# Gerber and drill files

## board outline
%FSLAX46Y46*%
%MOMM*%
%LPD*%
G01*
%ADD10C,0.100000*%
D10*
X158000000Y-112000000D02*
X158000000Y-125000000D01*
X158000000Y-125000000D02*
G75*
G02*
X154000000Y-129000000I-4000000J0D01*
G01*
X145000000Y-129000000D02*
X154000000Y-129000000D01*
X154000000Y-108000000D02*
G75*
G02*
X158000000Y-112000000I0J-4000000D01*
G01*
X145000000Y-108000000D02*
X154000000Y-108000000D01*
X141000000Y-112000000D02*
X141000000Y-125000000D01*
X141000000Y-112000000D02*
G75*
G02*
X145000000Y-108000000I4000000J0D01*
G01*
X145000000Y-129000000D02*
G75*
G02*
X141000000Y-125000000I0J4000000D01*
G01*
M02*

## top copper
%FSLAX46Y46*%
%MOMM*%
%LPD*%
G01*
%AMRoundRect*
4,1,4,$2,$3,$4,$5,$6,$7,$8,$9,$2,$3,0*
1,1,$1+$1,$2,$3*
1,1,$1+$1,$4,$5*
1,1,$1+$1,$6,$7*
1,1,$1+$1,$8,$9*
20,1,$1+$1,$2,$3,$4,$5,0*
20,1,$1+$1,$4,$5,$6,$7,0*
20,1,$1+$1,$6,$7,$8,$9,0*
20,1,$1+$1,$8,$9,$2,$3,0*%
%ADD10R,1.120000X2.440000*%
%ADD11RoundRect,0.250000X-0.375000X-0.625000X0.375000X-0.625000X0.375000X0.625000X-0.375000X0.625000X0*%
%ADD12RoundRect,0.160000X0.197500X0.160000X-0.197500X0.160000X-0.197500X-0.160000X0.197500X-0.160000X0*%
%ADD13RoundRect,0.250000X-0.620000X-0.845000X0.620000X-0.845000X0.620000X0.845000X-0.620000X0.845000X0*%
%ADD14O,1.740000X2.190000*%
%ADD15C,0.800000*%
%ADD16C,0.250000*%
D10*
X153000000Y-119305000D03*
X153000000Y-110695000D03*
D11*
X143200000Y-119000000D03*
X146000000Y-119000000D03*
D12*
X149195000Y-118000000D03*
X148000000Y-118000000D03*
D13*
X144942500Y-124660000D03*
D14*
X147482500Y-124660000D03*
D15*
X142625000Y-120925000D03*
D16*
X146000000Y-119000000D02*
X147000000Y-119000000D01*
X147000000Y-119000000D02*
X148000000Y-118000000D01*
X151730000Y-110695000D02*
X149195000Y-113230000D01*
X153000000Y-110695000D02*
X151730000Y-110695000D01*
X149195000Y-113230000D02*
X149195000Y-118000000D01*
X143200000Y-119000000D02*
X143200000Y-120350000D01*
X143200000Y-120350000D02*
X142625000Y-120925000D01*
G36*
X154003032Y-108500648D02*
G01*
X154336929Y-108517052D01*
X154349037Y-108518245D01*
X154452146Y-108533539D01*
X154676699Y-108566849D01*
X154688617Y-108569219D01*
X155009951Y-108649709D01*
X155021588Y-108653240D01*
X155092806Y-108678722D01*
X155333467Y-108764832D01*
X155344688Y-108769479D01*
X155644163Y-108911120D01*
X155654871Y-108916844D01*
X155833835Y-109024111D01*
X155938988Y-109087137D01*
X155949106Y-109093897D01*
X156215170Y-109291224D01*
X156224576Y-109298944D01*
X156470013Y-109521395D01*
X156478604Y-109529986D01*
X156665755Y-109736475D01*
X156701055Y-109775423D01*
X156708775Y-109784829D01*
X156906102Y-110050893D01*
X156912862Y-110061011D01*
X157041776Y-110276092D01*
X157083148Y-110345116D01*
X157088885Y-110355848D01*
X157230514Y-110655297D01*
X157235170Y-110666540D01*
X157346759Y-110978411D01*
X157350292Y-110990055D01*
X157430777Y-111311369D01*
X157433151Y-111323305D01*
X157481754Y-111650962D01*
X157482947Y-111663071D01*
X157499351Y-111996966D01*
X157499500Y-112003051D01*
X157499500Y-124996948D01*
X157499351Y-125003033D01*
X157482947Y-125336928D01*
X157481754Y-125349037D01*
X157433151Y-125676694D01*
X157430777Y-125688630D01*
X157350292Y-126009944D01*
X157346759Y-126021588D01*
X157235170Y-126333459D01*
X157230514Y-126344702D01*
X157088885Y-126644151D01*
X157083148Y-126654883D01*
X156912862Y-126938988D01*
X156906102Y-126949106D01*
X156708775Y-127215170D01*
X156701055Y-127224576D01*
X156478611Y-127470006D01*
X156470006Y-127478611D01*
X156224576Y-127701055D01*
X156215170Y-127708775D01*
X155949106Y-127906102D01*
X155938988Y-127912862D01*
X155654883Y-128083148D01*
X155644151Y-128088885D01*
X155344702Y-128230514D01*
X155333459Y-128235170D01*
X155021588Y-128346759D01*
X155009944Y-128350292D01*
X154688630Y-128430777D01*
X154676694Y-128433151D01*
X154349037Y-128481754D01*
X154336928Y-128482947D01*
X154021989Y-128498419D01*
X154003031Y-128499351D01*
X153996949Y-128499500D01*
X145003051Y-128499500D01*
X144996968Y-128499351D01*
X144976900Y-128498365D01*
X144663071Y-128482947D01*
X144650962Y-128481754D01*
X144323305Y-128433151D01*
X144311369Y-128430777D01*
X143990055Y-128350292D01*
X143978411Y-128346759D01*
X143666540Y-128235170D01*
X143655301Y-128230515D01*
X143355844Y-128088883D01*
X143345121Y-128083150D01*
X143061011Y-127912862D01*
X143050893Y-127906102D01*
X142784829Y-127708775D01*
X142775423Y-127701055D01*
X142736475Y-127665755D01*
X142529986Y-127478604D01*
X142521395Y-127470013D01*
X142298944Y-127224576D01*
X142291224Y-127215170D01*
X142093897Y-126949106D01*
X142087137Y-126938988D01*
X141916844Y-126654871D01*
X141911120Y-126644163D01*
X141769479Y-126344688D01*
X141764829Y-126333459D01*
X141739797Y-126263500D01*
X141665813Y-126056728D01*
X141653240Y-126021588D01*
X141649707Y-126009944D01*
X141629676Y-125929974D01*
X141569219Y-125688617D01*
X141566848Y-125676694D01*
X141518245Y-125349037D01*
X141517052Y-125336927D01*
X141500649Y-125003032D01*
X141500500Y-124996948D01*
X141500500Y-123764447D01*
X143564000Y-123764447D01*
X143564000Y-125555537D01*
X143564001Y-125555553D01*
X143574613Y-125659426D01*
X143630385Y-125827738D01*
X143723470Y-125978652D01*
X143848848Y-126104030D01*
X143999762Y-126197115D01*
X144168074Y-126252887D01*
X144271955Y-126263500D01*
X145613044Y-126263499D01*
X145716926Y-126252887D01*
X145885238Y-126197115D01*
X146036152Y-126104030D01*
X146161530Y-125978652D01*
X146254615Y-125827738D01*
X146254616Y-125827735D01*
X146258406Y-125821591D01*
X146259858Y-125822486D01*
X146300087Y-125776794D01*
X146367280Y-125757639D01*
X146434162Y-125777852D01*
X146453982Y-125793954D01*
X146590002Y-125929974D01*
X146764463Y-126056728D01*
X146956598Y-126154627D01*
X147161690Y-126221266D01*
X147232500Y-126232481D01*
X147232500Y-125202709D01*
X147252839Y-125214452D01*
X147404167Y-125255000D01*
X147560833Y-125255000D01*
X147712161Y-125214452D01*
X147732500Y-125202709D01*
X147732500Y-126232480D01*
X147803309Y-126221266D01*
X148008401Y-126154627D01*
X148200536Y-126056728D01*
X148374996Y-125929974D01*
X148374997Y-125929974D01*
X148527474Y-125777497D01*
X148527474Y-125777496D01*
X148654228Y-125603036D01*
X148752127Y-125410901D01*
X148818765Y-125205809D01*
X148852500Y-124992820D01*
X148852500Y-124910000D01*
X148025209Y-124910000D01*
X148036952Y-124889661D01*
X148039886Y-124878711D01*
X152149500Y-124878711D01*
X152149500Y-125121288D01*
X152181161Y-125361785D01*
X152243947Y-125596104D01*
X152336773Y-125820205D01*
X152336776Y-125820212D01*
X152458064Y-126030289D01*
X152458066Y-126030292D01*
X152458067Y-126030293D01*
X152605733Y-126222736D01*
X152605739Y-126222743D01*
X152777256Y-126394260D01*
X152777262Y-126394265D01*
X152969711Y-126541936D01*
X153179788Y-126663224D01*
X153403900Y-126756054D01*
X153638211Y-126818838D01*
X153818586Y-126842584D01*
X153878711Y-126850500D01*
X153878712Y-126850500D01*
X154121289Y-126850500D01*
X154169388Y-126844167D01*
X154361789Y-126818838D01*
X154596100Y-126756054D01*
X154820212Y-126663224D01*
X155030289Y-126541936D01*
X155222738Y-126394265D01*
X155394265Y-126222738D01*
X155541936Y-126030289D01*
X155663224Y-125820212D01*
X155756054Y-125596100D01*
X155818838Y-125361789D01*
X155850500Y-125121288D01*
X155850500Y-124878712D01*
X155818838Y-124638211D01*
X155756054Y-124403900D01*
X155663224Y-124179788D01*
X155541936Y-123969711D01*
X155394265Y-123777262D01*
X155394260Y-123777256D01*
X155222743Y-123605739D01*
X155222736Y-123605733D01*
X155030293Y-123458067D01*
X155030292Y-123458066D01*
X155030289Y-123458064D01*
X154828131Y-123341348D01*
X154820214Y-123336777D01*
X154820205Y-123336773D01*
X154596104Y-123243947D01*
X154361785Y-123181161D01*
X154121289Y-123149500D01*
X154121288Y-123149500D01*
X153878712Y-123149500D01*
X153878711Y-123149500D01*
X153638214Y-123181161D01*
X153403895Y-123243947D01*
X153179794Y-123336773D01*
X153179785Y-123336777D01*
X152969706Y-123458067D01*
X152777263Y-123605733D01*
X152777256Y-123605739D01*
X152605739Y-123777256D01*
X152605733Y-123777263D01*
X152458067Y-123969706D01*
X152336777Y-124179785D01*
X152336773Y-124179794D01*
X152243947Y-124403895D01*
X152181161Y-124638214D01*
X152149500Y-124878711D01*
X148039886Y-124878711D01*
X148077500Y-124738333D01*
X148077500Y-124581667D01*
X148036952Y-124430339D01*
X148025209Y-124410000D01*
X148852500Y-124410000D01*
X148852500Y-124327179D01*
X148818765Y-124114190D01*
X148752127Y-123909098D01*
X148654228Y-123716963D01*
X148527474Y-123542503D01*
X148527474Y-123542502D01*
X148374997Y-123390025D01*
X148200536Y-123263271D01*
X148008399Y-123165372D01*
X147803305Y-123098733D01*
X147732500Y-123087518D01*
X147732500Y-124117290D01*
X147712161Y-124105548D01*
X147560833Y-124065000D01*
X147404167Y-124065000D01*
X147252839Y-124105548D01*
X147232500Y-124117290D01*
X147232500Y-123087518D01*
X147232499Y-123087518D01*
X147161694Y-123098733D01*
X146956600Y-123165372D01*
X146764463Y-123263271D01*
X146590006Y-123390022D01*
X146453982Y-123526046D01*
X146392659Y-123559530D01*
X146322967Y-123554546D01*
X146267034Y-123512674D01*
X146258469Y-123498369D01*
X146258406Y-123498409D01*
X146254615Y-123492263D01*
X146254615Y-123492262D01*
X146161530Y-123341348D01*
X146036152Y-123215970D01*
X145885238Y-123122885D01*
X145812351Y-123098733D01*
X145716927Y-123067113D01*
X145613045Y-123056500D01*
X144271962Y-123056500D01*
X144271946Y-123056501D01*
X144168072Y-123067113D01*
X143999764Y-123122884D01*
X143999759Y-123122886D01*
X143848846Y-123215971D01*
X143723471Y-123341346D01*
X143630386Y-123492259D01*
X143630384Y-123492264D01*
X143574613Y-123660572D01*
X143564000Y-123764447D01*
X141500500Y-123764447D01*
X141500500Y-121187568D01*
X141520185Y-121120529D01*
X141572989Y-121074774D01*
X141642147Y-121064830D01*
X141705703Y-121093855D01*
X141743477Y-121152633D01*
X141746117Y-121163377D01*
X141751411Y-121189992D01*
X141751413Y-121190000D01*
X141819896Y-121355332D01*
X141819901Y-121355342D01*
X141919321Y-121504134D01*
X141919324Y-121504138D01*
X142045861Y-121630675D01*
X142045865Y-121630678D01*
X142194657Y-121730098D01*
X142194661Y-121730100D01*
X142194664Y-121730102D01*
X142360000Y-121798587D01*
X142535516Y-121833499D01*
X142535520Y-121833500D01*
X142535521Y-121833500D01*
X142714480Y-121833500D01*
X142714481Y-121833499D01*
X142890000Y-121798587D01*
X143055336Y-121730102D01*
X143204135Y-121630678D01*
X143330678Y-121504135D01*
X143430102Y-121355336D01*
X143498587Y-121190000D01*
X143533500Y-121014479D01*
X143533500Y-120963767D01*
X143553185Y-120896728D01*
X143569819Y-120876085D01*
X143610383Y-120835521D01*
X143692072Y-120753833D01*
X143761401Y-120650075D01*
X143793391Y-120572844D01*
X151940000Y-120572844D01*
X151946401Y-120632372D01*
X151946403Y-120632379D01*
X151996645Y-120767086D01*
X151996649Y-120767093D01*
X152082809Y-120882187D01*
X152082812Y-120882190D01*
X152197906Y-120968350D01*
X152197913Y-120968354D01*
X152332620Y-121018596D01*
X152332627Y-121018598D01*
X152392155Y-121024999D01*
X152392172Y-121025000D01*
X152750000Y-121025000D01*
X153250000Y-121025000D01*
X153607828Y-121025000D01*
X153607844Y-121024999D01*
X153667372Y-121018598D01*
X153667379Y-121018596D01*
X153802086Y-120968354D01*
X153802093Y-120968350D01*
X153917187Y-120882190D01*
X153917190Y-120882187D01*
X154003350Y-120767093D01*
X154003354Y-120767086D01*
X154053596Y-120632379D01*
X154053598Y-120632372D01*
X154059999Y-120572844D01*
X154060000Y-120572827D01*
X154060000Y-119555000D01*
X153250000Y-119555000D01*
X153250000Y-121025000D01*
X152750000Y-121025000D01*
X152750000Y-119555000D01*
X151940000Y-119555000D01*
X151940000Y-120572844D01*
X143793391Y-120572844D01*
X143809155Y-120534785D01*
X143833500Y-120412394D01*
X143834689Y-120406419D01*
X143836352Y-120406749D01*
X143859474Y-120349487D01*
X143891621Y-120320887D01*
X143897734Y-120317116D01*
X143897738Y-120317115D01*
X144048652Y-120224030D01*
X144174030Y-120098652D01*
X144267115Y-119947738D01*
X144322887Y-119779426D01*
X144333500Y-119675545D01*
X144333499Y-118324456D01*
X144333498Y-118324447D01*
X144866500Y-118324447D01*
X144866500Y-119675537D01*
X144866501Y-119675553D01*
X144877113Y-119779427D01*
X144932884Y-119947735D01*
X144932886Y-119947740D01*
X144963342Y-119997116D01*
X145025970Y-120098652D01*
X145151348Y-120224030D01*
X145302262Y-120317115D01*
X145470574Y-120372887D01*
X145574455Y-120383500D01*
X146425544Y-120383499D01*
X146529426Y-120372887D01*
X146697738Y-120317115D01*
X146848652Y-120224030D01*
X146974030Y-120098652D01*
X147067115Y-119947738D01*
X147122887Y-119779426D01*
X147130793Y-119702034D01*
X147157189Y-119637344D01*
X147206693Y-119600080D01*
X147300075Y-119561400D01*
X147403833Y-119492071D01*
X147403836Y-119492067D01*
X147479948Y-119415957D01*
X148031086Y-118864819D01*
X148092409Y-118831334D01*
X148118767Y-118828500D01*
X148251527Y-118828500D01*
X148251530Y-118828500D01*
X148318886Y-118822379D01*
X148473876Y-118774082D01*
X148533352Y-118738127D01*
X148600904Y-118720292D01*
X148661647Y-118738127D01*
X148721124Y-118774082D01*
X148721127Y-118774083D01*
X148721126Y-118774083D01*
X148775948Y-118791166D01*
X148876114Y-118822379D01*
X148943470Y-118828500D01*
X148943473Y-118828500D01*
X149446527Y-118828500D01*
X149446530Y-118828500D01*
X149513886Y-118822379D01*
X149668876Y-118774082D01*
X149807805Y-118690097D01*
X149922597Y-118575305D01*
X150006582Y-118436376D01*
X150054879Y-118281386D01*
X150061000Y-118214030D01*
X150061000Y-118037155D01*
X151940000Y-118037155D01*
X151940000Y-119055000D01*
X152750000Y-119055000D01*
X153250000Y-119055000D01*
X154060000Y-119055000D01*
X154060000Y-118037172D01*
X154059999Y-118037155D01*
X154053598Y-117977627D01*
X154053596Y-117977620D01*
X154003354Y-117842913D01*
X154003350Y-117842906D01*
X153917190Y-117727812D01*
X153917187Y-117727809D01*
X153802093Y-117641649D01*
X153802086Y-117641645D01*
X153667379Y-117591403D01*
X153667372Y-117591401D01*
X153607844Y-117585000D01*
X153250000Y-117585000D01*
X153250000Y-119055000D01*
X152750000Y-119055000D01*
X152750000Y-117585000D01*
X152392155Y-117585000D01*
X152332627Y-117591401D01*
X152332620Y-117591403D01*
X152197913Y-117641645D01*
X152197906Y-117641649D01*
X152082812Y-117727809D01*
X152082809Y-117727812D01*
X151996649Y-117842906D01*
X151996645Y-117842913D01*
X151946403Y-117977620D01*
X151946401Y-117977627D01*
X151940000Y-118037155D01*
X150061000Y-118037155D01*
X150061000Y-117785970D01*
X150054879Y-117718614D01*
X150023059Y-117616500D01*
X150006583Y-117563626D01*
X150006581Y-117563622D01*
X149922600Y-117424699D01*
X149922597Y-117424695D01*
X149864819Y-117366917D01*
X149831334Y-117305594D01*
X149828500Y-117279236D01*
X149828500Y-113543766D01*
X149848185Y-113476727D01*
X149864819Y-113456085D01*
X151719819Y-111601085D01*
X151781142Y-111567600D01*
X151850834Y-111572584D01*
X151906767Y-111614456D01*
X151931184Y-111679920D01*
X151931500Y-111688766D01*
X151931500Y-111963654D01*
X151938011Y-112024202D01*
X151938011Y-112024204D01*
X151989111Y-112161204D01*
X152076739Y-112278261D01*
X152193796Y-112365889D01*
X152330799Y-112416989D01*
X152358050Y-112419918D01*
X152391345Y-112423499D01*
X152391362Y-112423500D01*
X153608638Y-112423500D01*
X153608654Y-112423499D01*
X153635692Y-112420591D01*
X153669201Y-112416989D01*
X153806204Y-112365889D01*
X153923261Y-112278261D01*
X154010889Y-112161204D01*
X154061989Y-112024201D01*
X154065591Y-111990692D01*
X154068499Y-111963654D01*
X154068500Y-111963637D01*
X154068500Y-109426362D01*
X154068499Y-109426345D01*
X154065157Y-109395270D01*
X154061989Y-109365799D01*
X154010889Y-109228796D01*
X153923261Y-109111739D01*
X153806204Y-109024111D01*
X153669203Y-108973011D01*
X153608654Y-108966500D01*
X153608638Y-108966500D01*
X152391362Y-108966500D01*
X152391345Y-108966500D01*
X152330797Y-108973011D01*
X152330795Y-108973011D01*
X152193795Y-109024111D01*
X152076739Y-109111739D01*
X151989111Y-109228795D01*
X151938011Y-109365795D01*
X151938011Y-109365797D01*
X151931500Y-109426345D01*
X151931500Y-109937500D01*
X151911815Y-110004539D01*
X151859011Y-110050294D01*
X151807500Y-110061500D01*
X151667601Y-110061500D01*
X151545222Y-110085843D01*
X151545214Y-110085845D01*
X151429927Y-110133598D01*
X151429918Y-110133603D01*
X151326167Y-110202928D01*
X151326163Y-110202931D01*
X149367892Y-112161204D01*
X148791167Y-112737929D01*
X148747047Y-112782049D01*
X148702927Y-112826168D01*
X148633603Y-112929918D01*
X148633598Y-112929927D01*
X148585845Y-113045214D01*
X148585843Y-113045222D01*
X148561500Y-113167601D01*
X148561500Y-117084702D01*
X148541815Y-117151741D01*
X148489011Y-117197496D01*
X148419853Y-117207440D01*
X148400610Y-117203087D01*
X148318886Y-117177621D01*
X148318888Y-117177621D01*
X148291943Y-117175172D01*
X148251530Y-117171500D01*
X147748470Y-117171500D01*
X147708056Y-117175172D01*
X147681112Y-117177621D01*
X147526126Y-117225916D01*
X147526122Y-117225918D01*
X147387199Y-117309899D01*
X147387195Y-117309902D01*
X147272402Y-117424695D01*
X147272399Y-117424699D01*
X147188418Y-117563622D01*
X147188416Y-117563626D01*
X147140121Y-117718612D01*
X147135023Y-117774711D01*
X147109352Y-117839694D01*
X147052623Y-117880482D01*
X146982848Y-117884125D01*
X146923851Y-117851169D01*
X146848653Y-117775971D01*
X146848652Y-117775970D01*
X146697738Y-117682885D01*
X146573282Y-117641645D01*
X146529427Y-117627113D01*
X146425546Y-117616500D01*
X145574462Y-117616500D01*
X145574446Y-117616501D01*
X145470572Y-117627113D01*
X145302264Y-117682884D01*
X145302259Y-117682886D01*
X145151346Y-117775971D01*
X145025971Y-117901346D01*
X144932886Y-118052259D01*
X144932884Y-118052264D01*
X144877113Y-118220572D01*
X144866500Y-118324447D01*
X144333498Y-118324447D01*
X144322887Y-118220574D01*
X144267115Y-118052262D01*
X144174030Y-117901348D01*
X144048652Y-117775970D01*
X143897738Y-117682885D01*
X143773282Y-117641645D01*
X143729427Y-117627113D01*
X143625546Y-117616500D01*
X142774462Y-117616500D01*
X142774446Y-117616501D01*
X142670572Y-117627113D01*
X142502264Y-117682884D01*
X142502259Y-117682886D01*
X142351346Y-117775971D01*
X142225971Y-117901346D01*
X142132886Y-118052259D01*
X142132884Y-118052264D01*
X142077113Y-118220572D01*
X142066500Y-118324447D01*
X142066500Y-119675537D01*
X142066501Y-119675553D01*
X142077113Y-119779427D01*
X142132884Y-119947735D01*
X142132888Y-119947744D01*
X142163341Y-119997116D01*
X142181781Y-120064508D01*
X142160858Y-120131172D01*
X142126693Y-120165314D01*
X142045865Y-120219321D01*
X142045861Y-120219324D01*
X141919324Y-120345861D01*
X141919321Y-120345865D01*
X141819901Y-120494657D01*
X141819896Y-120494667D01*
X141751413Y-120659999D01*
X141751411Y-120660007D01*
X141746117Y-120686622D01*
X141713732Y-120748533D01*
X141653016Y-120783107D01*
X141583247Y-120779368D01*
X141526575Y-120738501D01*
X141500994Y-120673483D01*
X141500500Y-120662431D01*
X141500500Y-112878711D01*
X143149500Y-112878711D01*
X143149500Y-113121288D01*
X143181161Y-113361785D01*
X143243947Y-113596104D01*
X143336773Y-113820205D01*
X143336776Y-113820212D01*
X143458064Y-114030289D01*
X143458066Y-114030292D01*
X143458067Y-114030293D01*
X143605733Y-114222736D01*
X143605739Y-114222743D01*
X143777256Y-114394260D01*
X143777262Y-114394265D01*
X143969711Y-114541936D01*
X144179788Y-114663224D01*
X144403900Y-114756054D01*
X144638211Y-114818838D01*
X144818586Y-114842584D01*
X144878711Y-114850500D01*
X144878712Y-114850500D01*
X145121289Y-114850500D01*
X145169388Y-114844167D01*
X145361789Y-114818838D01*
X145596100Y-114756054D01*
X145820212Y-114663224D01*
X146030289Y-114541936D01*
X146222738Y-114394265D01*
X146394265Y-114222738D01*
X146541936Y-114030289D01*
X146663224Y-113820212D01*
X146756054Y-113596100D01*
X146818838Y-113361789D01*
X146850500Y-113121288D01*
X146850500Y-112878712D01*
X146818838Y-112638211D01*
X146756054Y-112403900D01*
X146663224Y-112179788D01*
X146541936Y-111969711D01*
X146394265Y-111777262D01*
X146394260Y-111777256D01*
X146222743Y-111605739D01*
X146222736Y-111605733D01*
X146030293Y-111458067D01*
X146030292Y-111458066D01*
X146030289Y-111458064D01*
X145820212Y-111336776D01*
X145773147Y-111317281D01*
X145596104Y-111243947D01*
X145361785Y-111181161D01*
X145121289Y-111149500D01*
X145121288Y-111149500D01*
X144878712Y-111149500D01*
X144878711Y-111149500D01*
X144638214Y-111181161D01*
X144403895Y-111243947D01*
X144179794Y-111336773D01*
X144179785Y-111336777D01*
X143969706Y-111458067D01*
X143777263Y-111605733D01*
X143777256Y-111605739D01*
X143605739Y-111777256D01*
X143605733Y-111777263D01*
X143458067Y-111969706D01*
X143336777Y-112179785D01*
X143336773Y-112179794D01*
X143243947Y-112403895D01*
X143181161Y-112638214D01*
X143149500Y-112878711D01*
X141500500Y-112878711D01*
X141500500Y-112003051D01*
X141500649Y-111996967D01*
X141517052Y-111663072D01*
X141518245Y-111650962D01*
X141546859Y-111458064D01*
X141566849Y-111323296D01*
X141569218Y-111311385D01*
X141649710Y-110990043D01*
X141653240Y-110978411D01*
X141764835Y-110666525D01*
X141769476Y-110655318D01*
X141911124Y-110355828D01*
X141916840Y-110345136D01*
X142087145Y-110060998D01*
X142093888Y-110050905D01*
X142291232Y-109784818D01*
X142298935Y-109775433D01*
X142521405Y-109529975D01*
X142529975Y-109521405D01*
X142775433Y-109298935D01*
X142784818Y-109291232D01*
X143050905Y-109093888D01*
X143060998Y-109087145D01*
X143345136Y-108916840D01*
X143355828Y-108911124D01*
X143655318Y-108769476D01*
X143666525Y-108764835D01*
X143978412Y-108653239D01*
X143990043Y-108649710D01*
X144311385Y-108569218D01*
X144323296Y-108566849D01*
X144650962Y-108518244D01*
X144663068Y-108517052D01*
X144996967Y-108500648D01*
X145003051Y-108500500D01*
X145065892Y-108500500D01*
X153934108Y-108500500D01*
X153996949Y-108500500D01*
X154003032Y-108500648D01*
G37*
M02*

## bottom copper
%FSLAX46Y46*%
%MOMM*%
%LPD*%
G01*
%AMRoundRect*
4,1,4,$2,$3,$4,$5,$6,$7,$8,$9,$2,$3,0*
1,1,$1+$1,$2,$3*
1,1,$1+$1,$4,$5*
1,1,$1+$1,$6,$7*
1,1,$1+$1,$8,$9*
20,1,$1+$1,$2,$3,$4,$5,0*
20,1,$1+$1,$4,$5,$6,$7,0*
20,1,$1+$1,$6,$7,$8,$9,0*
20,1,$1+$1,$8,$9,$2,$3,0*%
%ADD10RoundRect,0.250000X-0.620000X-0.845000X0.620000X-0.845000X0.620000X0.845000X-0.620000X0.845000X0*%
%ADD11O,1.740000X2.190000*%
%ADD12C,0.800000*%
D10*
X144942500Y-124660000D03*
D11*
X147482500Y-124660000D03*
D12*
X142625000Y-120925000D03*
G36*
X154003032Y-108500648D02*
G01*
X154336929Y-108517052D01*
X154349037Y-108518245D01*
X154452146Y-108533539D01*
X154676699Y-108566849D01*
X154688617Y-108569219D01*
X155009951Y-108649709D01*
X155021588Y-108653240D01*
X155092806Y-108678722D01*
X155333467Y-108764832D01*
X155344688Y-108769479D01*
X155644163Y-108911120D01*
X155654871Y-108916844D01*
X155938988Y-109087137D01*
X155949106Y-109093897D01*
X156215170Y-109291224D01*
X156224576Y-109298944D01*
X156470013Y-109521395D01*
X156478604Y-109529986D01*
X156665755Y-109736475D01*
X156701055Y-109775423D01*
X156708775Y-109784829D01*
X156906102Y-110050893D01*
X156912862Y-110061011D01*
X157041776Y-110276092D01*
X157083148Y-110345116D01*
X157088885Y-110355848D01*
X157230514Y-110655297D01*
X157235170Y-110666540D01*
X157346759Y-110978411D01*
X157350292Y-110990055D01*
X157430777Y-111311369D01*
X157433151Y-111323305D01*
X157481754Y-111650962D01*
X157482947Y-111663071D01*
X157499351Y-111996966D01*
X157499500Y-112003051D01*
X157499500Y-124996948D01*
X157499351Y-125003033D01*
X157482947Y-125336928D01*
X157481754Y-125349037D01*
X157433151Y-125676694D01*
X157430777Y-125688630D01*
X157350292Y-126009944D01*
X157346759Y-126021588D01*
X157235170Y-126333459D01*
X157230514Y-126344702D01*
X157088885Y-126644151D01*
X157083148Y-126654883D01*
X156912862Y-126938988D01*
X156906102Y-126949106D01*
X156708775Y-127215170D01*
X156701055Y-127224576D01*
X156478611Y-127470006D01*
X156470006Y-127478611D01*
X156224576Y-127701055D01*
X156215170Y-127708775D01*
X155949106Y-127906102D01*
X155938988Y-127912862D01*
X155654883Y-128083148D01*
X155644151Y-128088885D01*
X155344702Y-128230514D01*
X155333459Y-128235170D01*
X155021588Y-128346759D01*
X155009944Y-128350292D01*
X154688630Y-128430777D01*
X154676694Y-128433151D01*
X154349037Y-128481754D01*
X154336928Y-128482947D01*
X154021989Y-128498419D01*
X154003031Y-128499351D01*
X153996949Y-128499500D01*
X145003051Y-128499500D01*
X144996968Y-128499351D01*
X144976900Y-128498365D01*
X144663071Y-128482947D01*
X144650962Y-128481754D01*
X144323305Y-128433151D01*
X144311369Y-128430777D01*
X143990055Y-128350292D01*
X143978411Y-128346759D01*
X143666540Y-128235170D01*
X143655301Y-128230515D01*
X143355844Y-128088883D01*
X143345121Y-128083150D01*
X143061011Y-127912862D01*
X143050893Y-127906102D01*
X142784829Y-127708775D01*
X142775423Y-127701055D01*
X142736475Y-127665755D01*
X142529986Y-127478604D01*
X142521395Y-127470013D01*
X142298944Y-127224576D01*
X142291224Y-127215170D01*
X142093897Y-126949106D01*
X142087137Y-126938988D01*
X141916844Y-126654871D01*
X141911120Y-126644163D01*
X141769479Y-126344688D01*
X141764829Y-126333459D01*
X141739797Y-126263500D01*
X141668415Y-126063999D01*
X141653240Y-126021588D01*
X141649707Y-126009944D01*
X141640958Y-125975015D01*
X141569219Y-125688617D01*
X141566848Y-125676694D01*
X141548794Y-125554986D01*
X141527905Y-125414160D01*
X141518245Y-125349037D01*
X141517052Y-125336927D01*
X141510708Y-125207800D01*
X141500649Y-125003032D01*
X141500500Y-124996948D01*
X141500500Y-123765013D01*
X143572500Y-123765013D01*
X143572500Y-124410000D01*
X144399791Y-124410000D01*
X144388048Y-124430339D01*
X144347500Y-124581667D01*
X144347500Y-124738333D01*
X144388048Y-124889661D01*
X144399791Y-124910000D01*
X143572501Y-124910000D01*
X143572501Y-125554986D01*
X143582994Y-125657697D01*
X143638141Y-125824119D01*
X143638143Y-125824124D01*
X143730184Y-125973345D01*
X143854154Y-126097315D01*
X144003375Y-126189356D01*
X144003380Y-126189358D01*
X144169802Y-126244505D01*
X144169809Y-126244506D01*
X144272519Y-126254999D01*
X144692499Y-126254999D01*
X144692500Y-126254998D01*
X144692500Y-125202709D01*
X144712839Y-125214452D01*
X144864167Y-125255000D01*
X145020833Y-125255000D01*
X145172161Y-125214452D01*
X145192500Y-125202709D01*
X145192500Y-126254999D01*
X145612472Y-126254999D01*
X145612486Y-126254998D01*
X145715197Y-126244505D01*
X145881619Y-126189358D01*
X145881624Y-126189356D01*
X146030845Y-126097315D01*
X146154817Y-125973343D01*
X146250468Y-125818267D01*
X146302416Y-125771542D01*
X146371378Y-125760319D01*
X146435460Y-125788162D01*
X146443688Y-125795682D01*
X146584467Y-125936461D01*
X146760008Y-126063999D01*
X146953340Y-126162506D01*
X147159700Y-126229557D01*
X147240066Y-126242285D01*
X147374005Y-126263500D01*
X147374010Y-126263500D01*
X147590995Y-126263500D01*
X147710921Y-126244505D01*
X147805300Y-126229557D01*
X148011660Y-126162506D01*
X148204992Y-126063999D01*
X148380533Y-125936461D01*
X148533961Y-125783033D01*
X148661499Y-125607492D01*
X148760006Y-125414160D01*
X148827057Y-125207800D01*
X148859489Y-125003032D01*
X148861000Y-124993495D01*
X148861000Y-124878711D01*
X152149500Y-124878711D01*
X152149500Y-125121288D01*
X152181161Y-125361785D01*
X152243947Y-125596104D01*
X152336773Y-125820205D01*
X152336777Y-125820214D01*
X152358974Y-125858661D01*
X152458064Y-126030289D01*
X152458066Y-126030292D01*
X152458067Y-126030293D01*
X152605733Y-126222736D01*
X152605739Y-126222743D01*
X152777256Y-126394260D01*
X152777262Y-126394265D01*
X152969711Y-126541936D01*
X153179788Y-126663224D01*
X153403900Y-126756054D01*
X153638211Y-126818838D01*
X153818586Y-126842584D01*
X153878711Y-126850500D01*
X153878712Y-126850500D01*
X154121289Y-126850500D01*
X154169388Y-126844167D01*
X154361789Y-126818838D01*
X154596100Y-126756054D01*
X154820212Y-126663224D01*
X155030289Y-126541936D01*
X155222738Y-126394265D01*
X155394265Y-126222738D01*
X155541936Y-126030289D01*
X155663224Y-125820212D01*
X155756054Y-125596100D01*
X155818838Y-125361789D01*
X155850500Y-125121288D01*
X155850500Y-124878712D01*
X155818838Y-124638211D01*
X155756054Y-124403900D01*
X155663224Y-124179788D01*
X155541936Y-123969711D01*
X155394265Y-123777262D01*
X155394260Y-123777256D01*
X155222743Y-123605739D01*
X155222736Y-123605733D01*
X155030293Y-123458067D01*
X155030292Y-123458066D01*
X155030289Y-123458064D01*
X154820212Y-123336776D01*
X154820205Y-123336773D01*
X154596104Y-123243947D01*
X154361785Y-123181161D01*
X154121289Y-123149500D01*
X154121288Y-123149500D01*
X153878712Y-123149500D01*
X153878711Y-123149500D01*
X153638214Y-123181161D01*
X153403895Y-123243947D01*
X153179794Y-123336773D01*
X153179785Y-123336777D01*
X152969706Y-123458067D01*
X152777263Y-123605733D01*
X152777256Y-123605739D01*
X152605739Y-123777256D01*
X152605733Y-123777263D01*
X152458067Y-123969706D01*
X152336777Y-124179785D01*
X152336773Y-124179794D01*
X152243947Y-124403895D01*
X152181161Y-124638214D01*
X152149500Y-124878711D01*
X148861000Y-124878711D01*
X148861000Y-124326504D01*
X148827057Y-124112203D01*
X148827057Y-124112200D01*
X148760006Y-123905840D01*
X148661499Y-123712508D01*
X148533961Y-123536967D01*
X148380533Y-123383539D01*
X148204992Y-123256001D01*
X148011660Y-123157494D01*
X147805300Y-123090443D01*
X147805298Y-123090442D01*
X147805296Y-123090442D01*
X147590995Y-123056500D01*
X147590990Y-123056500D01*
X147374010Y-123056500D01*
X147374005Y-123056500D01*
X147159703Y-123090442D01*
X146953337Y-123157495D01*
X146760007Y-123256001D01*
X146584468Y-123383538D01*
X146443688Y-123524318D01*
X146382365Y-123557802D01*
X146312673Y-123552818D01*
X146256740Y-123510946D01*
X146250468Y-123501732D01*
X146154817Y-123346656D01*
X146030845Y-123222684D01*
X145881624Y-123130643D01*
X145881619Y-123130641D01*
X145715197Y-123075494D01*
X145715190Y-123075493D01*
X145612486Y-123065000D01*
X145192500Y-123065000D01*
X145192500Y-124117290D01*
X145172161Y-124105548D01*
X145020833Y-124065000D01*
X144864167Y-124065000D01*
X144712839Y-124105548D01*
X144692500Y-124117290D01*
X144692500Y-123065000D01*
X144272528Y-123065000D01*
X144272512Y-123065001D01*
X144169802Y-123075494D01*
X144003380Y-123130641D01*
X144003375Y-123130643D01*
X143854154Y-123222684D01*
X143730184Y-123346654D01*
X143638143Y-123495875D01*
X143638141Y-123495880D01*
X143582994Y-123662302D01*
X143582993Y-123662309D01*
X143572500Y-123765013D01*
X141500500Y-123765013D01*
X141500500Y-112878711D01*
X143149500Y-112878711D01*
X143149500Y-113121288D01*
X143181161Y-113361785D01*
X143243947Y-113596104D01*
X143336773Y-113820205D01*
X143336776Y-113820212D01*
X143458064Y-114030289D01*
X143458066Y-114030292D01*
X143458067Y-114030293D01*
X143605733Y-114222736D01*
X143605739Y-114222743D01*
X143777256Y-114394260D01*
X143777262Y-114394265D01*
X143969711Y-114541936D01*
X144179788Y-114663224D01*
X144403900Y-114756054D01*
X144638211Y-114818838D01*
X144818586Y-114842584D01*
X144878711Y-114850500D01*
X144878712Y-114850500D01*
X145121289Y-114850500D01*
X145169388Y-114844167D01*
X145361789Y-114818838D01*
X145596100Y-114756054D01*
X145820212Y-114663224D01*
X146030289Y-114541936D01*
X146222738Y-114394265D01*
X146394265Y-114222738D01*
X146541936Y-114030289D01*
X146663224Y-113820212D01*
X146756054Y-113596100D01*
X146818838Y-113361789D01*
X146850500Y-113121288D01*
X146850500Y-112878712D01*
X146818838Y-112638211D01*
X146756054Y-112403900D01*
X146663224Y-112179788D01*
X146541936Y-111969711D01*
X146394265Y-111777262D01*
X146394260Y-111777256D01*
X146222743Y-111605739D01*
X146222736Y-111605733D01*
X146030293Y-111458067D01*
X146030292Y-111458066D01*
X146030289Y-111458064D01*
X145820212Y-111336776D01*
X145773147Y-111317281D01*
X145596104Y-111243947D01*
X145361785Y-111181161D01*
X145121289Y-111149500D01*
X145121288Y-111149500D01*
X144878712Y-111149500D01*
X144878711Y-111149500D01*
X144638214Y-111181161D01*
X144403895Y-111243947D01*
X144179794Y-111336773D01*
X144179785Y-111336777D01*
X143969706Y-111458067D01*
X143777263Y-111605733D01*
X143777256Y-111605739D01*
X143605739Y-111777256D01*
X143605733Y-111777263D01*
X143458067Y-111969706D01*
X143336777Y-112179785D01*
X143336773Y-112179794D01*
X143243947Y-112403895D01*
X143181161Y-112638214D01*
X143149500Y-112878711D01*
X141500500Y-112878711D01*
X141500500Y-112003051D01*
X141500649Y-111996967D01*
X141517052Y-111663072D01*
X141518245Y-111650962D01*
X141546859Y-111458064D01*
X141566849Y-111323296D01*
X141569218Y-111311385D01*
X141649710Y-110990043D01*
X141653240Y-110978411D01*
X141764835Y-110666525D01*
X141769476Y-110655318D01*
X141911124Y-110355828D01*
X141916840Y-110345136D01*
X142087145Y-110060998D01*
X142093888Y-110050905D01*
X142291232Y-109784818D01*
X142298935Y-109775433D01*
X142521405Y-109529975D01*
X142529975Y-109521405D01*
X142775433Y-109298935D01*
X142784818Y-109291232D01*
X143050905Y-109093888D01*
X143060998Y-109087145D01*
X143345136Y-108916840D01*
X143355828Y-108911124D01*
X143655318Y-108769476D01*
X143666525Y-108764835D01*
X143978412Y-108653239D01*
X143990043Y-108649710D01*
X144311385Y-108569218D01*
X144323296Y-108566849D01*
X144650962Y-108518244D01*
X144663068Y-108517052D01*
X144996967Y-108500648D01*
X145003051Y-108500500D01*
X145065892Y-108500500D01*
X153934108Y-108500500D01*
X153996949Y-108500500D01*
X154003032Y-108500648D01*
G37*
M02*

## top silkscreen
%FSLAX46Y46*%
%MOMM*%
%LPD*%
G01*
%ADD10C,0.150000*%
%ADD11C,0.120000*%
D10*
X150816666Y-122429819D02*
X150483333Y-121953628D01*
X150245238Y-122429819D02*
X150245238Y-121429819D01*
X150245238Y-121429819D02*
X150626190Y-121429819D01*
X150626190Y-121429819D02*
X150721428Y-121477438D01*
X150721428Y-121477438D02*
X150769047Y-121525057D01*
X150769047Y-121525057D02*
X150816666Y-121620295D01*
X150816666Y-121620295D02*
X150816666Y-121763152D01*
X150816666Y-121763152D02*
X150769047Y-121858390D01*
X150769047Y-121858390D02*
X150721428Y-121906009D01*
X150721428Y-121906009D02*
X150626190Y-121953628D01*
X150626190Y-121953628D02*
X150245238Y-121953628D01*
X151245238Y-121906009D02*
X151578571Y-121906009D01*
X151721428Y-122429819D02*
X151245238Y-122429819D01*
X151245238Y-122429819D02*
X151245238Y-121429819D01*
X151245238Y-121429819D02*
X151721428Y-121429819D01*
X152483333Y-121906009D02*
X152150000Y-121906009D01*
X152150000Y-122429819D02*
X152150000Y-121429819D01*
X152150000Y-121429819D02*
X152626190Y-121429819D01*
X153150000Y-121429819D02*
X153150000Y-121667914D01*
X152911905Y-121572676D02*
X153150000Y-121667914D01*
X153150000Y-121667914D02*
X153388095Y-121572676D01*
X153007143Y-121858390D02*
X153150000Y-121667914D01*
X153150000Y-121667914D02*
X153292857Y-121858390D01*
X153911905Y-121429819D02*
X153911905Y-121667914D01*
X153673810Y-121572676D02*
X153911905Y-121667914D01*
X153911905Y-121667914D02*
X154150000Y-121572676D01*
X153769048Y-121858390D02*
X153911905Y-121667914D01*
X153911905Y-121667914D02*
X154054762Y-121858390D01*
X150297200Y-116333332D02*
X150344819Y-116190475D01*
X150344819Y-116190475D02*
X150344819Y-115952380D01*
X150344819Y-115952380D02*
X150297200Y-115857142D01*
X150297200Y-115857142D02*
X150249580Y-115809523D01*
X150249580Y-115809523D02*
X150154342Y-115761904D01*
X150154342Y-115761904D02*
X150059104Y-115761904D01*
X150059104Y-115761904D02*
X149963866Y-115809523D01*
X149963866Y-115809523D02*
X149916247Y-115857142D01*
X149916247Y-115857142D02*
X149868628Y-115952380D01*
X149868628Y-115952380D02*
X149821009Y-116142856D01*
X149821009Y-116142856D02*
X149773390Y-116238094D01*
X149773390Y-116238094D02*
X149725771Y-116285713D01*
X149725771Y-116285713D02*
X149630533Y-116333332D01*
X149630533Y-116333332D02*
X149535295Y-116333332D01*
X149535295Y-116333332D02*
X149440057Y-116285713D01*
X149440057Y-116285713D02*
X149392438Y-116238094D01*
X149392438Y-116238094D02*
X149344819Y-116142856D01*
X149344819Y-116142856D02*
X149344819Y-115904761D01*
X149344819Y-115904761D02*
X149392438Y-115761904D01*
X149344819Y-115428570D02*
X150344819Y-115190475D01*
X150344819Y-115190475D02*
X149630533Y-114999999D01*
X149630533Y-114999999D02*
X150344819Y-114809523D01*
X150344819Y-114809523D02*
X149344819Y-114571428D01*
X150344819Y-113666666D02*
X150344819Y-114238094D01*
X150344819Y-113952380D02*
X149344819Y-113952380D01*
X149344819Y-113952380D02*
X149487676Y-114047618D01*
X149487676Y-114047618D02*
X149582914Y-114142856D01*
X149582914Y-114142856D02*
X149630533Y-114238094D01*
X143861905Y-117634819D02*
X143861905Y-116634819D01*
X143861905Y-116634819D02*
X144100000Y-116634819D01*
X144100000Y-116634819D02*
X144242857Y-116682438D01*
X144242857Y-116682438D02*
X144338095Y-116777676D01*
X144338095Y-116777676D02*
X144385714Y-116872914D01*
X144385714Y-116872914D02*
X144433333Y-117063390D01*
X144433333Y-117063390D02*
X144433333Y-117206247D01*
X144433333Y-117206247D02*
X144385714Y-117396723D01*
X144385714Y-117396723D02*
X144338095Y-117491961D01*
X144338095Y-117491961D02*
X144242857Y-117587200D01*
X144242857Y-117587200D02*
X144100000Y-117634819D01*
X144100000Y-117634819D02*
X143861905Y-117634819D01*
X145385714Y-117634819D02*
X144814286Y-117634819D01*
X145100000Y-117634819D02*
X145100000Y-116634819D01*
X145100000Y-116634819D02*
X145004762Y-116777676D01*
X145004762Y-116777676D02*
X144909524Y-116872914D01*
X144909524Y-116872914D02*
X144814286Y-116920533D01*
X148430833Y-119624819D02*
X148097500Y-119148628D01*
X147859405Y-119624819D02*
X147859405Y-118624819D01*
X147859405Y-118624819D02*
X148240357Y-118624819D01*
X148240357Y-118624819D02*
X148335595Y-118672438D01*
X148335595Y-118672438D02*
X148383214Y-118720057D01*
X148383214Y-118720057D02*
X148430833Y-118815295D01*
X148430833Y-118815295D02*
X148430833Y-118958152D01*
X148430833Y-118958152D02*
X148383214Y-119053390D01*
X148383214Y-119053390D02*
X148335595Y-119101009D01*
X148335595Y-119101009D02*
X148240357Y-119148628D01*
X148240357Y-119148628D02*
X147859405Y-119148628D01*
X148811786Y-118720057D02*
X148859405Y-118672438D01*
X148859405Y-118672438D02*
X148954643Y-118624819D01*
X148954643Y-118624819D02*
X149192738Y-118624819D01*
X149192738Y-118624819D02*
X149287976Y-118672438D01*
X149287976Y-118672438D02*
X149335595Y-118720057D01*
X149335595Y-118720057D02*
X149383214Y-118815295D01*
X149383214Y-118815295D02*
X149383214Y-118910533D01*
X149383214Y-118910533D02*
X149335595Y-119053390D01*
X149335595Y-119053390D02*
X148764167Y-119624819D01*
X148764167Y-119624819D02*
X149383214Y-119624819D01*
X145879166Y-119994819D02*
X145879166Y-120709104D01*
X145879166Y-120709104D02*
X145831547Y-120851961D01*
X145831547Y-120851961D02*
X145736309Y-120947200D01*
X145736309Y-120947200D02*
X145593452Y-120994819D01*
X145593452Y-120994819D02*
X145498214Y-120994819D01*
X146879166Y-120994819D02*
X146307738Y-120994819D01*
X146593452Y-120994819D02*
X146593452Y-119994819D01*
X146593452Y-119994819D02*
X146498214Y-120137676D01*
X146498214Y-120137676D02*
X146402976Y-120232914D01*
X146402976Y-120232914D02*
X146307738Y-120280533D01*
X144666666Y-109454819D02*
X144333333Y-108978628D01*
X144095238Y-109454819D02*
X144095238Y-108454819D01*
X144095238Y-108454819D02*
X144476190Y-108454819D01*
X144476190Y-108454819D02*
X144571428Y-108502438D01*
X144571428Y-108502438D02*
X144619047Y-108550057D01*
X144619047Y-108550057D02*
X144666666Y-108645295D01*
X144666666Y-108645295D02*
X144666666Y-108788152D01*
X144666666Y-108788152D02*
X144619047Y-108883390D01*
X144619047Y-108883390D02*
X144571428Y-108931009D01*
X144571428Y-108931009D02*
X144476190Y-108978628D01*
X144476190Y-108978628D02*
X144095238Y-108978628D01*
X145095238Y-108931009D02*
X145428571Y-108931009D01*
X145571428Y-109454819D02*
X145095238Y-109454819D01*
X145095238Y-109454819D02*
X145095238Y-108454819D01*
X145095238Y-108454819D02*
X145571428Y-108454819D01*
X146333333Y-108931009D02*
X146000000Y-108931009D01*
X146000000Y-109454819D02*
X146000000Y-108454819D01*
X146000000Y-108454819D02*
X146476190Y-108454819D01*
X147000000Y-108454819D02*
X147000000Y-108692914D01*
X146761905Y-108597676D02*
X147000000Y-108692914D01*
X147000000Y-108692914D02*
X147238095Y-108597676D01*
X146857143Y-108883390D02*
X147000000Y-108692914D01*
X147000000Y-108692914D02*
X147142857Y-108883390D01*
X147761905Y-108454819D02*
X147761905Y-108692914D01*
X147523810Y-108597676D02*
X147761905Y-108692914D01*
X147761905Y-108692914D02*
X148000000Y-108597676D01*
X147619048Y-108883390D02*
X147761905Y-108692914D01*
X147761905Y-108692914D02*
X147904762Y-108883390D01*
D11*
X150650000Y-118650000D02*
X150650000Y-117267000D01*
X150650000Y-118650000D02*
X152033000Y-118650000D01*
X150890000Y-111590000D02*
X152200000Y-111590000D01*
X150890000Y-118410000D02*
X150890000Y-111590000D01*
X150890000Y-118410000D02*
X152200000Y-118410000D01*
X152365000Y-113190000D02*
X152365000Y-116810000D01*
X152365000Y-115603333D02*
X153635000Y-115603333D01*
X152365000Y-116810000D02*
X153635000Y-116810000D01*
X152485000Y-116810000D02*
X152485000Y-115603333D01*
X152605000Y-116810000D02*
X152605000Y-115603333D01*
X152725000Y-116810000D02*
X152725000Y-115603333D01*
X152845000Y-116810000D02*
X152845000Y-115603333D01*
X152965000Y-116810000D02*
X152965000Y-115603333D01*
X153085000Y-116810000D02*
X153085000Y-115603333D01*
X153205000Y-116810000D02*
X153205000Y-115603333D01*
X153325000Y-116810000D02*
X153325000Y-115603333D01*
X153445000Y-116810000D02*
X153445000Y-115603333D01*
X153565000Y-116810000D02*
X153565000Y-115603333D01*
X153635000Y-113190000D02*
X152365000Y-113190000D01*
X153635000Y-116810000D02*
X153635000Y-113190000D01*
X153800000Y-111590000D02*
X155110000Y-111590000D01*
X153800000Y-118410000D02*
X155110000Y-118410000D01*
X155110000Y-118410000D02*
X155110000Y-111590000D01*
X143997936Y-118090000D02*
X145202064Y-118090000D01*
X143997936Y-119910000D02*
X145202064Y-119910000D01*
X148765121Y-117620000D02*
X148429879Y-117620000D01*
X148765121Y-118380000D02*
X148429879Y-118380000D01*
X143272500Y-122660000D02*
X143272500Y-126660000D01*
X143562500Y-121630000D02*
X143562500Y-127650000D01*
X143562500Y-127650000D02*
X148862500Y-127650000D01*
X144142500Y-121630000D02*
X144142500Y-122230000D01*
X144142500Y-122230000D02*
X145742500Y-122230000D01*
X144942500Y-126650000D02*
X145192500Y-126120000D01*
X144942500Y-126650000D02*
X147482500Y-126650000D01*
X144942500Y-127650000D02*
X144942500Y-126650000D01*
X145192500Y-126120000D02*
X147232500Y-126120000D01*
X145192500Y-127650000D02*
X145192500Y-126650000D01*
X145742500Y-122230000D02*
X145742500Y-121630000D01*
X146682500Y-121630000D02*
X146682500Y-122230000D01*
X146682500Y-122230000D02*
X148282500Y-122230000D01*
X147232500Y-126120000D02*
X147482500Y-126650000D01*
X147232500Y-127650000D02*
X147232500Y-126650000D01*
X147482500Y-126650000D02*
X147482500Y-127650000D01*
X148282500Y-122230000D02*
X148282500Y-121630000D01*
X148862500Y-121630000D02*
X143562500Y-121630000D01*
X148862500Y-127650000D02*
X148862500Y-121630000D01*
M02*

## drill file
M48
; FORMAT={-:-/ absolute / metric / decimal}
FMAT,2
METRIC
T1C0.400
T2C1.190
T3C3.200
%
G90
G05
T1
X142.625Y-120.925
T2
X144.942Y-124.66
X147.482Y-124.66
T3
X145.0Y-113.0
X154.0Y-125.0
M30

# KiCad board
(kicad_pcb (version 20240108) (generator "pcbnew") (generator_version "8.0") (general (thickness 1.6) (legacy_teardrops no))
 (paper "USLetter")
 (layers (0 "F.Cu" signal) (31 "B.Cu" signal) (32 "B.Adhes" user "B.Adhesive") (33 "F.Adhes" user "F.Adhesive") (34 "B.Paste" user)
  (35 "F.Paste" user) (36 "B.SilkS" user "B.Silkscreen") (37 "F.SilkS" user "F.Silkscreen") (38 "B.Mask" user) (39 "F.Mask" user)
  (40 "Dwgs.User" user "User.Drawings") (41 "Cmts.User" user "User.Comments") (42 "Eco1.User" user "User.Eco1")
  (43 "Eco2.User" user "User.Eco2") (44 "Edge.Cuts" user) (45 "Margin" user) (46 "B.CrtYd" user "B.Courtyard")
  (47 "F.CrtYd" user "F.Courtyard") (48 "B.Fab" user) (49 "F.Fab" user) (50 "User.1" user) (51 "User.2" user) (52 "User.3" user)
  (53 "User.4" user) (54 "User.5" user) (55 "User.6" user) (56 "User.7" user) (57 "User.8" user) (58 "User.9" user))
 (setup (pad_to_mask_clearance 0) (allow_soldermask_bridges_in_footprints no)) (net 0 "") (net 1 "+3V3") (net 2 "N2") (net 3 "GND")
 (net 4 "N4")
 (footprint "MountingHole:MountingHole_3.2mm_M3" (layer "F.Cu") (at 154 125)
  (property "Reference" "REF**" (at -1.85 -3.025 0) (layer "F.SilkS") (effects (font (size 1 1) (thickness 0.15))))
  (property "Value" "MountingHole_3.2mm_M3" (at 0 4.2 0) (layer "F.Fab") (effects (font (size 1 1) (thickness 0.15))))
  (pad "" np_thru_hole circle (at 0 0) (size 3.2 3.2) (drill 3.2) (layers "*.Cu" "*.Mask")))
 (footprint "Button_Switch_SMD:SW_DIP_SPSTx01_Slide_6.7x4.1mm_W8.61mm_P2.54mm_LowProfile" (layer "F.Cu") (at 153 115 90)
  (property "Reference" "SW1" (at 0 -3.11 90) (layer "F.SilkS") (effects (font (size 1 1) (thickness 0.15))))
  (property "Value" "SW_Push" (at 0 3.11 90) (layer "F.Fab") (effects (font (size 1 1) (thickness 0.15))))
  (fp_line (start -3.65 -2.35) (end -2.267 -2.35) (stroke (width 0.12) (type solid)) (layer "F.SilkS"))
  (fp_line (start -3.65 -2.35) (end -3.65 -0.967) (stroke (width 0.12) (type solid)) (layer "F.SilkS"))
  (fp_line (start 3.41 -2.11) (end 3.41 -0.8) (stroke (width 0.12) (type solid)) (layer "F.SilkS"))
  (fp_line (start -3.41 -2.11) (end 3.41 -2.11) (stroke (width 0.12) (type solid)) (layer "F.SilkS"))
  (fp_line (start -3.41 -2.11) (end -3.41 -0.8) (stroke (width 0.12) (type solid)) (layer "F.SilkS"))
  (fp_line (start 1.81 -0.635) (end -1.81 -0.635) (stroke (width 0.12) (type solid)) (layer "F.SilkS"))
  (fp_line (start -0.603333 -0.635) (end -0.603333 0.635) (stroke (width 0.12) (type solid)) (layer "F.SilkS"))
  (fp_line (start -1.81 -0.635) (end -1.81 0.635) (stroke (width 0.12) (type solid)) (layer "F.SilkS"))
  (fp_line (start -1.81 -0.515) (end -0.603333 -0.515) (stroke (width 0.12) (type solid)) (layer "F.SilkS"))
  (fp_line (start -1.81 -0.395) (end -0.603333 -0.395) (stroke (width 0.12) (type solid)) (layer "F.SilkS"))
  (fp_line (start -1.81 -0.275) (end -0.603333 -0.275) (stroke (width 0.12) (type solid)) (layer "F.SilkS"))
  (fp_line (start -1.81 -0.155) (end -0.603333 -0.155) (stroke (width 0.12) (type solid)) (layer "F.SilkS"))
  (fp_line (start -1.81 -0.035) (end -0.603333 -0.035) (stroke (width 0.12) (type solid)) (layer "F.SilkS"))
  (fp_line (start -1.81 0.085) (end -0.603333 0.085) (stroke (width 0.12) (type solid)) (layer "F.SilkS"))
  (fp_line (start -1.81 0.205) (end -0.603333 0.205) (stroke (width 0.12) (type solid)) (layer "F.SilkS"))
  (fp_line (start -1.81 0.325) (end -0.603333 0.325) (stroke (width 0.12) (type solid)) (layer "F.SilkS"))
  (fp_line (start -1.81 0.445) (end -0.603333 0.445) (stroke (width 0.12) (type solid)) (layer "F.SilkS"))
  (fp_line (start -1.81 0.565) (end -0.603333 0.565) (stroke (width 0.12) (type solid)) (layer "F.SilkS"))
  (fp_line (start 1.81 0.635) (end 1.81 -0.635) (stroke (width 0.12) (type solid)) (layer "F.SilkS"))
  (fp_line (start -1.81 0.635) (end 1.81 0.635) (stroke (width 0.12) (type solid)) (layer "F.SilkS"))
  (fp_line (start 3.41 0.8) (end 3.41 2.11) (stroke (width 0.12) (type solid)) (layer "F.SilkS"))
  (fp_line (start -3.41 0.8) (end -3.41 2.11) (stroke (width 0.12) (type solid)) (layer "F.SilkS"))
  (fp_line (start -3.41 2.11) (end 3.41 2.11) (stroke (width 0.12) (type solid)) (layer "F.SilkS"))
  (pad "1" smd rect (at -4.305 0 90) (size 2.44 1.12) (layers "F.Cu" "F.Paste" "F.Mask") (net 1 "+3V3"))
  (pad "2" smd rect (at 4.305 0 90) (size 2.44 1.12) (layers "F.Cu" "F.Paste" "F.Mask") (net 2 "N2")))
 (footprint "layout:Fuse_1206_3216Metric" (layer "F.Cu") (at 144.6 119)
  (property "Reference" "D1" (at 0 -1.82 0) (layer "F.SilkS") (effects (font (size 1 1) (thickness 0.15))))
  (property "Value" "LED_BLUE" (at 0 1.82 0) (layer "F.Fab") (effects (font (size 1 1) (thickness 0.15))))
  (fp_line (start -0.602064 -0.91) (end 0.602064 -0.91) (stroke (width 0.12) (type solid)) (layer "F.SilkS"))
  (fp_line (start -0.602064 0.91) (end 0.602064 0.91) (stroke (width 0.12) (type solid)) (layer "F.SilkS"))
  (pad "1" smd roundrect (at -1.4 0) (size 1.25 1.75) (layers "F.Cu" "F.Paste" "F.Mask") (roundrect_rratio 0.2) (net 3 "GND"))
  (pad "2" smd roundrect (at 1.4 0) (size 1.25 1.75) (layers "F.Cu" "F.Paste" "F.Mask") (roundrect_rratio 0.2) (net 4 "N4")))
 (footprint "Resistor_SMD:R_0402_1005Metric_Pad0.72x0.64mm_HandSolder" (layer "F.Cu") (at 148.5975 118 180)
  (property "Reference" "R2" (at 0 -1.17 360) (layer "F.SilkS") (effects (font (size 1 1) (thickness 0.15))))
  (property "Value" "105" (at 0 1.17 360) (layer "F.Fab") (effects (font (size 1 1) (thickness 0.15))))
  (fp_line (start -0.167621 0.38) (end 0.167621 0.38) (stroke (width 0.12) (type solid)) (layer "F.SilkS"))
  (fp_line (start -0.167621 -0.38) (end 0.167621 -0.38) (stroke (width 0.12) (type solid)) (layer "F.SilkS"))
  (pad "1" smd roundrect (at -0.5975 0 180) (size 0.715 0.64) (layers "F.Cu" "F.Paste" "F.Mask") (roundrect_rratio 0.25) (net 2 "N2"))
  (pad "2" smd roundrect (at 0.5975 0 180) (size 0.715 0.64) (layers "F.Cu" "F.Paste" "F.Mask") (roundrect_rratio 0.25) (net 4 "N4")))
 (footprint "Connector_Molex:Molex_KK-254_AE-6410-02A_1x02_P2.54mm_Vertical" (layer "F.Cu") (at 144.9425 124.66)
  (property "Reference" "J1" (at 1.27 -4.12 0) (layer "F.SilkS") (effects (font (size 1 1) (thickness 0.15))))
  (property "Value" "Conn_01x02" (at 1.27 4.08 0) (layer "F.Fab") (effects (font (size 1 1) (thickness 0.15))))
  (fp_line (start -1.67 -2) (end -1.67 2) (stroke (width 0.12) (type solid)) (layer "F.SilkS"))
  (fp_line (start -1.38 -3.03) (end -1.38 2.99) (stroke (width 0.12) (type solid)) (layer "F.SilkS"))
  (fp_line (start -1.38 2.99) (end 3.92 2.99) (stroke (width 0.12) (type solid)) (layer "F.SilkS"))
  (fp_line (start -0.8 -3.03) (end -0.8 -2.43) (stroke (width 0.12) (type solid)) (layer "F.SilkS"))
  (fp_line (start -0.8 -2.43) (end 0.8 -2.43) (stroke (width 0.12) (type solid)) (layer "F.SilkS"))
  (fp_line (start 0 1.99) (end 0.25 1.46) (stroke (width 0.12) (type solid)) (layer "F.SilkS"))
  (fp_line (start 0 1.99) (end 2.54 1.99) (stroke (width 0.12) (type solid)) (layer "F.SilkS"))
  (fp_line (start 0 2.99) (end 0 1.99) (stroke (width 0.12) (type solid)) (layer "F.SilkS"))
  (fp_line (start 0.25 1.46) (end 2.29 1.46) (stroke (width 0.12) (type solid)) (layer "F.SilkS"))
  (fp_line (start 0.25 2.99) (end 0.25 1.99) (stroke (width 0.12) (type solid)) (layer "F.SilkS"))
  (fp_line (start 0.8 -2.43) (end 0.8 -3.03) (stroke (width 0.12) (type solid)) (layer "F.SilkS"))
  (fp_line (start 1.74 -3.03) (end 1.74 -2.43) (stroke (width 0.12) (type solid)) (layer "F.SilkS"))
  (fp_line (start 1.74 -2.43) (end 3.34 -2.43) (stroke (width 0.12) (type solid)) (layer "F.SilkS"))
  (fp_line (start 2.29 1.46) (end 2.54 1.99) (stroke (width 0.12) (type solid)) (layer "F.SilkS"))
  (fp_line (start 2.29 2.99) (end 2.29 1.99) (stroke (width 0.12) (type solid)) (layer "F.SilkS"))
  (fp_line (start 2.54 1.99) (end 2.54 2.99) (stroke (width 0.12) (type solid)) (layer "F.SilkS"))
  (fp_line (start 3.34 -2.43) (end 3.34 -3.03) (stroke (width 0.12) (type solid)) (layer "F.SilkS"))
  (fp_line (start 3.92 -3.03) (end -1.38 -3.03) (stroke (width 0.12) (type solid)) (layer "F.SilkS"))
  (fp_line (start 3.92 2.99) (end 3.92 -3.03) (stroke (width 0.12) (type solid)) (layer "F.SilkS"))
  (pad "1" thru_hole roundrect (at 0 0) (size 1.74 2.19) (drill 1.19) (layers "*.Cu" "*.Mask") (remove_unused_layers no)
   (roundrect_rratio 0.143678) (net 3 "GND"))
  (pad "2" thru_hole oval (at 2.54 0) (size 1.74 2.19) (drill 1.19) (layers "*.Cu" "*.Mask") (remove_unused_layers no) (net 1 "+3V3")))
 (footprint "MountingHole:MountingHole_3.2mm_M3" (layer "F.Cu") (at 145 113)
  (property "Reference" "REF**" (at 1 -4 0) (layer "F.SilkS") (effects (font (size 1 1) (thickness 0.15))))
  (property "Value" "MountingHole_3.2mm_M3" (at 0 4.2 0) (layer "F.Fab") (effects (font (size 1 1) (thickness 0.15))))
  (pad "" np_thru_hole circle (at 0 0) (size 3.2 3.2) (drill 3.2) (layers "*.Cu" "*.Mask")))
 (gr_line (start 158 112) (end 158 125) (stroke (width 0.1) (type default)) (layer "Edge.Cuts"))
 (gr_arc (start 158 125) (mid 156.828427 127.828427) (end 154 129) (stroke (width 0.1) (type default)) (layer "Edge.Cuts"))
 (gr_line (start 145 129) (end 154 129) (stroke (width 0.1) (type default)) (layer "Edge.Cuts"))
 (gr_arc (start 154 108) (mid 156.828427 109.171573) (end 158 112) (stroke (width 0.1) (type default)) (layer "Edge.Cuts"))
 (gr_line (start 145 108) (end 154 108) (stroke (width 0.1) (type default)) (layer "Edge.Cuts"))
 (gr_line (start 141 112) (end 141 125) (stroke (width 0.1) (type default)) (layer "Edge.Cuts"))
 (gr_arc (start 141 112) (mid 142.171573 109.171573) (end 145 108) (stroke (width 0.1) (type default)) (layer "Edge.Cuts"))
 (gr_arc (start 145 129) (mid 142.171573 127.828427) (end 141 125) (stroke (width 0.1) (type default)) (layer "Edge.Cuts"))
 (segment (start 146 119) (end 147 119) (width 0.25) (layer "F.Cu") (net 4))
 (segment (start 147 119) (end 148 118) (width 0.25) (layer "F.Cu") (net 4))
 (segment (start 151.73 110.695) (end 149.195 113.23) (width 0.25) (layer "F.Cu") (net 2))
 (segment (start 153 110.695) (end 151.73 110.695) (width 0.25) (layer "F.Cu") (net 2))
 (segment (start 149.195 113.23) (end 149.195 118) (width 0.25) (layer "F.Cu") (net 2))
 (segment (start 143.2 119) (end 143.2 120.35) (width 0.25) (layer "F.Cu") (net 3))
 (segment (start 143.2 120.35) (end 142.625 120.925) (width 0.25) (layer "F.Cu") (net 3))
 (via (at 142.625 120.925) (size 0.8) (drill 0.4) (layers "F.Cu" "B.Cu") (free yes) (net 3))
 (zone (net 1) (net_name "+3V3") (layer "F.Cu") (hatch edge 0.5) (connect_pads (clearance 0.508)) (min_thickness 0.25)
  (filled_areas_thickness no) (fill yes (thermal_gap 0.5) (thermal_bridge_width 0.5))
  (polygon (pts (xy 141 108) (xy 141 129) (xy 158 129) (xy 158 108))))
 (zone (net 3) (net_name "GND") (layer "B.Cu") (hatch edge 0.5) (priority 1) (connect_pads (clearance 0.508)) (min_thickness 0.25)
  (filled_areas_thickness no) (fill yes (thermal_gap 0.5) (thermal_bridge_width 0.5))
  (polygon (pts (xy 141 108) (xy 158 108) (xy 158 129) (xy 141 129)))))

